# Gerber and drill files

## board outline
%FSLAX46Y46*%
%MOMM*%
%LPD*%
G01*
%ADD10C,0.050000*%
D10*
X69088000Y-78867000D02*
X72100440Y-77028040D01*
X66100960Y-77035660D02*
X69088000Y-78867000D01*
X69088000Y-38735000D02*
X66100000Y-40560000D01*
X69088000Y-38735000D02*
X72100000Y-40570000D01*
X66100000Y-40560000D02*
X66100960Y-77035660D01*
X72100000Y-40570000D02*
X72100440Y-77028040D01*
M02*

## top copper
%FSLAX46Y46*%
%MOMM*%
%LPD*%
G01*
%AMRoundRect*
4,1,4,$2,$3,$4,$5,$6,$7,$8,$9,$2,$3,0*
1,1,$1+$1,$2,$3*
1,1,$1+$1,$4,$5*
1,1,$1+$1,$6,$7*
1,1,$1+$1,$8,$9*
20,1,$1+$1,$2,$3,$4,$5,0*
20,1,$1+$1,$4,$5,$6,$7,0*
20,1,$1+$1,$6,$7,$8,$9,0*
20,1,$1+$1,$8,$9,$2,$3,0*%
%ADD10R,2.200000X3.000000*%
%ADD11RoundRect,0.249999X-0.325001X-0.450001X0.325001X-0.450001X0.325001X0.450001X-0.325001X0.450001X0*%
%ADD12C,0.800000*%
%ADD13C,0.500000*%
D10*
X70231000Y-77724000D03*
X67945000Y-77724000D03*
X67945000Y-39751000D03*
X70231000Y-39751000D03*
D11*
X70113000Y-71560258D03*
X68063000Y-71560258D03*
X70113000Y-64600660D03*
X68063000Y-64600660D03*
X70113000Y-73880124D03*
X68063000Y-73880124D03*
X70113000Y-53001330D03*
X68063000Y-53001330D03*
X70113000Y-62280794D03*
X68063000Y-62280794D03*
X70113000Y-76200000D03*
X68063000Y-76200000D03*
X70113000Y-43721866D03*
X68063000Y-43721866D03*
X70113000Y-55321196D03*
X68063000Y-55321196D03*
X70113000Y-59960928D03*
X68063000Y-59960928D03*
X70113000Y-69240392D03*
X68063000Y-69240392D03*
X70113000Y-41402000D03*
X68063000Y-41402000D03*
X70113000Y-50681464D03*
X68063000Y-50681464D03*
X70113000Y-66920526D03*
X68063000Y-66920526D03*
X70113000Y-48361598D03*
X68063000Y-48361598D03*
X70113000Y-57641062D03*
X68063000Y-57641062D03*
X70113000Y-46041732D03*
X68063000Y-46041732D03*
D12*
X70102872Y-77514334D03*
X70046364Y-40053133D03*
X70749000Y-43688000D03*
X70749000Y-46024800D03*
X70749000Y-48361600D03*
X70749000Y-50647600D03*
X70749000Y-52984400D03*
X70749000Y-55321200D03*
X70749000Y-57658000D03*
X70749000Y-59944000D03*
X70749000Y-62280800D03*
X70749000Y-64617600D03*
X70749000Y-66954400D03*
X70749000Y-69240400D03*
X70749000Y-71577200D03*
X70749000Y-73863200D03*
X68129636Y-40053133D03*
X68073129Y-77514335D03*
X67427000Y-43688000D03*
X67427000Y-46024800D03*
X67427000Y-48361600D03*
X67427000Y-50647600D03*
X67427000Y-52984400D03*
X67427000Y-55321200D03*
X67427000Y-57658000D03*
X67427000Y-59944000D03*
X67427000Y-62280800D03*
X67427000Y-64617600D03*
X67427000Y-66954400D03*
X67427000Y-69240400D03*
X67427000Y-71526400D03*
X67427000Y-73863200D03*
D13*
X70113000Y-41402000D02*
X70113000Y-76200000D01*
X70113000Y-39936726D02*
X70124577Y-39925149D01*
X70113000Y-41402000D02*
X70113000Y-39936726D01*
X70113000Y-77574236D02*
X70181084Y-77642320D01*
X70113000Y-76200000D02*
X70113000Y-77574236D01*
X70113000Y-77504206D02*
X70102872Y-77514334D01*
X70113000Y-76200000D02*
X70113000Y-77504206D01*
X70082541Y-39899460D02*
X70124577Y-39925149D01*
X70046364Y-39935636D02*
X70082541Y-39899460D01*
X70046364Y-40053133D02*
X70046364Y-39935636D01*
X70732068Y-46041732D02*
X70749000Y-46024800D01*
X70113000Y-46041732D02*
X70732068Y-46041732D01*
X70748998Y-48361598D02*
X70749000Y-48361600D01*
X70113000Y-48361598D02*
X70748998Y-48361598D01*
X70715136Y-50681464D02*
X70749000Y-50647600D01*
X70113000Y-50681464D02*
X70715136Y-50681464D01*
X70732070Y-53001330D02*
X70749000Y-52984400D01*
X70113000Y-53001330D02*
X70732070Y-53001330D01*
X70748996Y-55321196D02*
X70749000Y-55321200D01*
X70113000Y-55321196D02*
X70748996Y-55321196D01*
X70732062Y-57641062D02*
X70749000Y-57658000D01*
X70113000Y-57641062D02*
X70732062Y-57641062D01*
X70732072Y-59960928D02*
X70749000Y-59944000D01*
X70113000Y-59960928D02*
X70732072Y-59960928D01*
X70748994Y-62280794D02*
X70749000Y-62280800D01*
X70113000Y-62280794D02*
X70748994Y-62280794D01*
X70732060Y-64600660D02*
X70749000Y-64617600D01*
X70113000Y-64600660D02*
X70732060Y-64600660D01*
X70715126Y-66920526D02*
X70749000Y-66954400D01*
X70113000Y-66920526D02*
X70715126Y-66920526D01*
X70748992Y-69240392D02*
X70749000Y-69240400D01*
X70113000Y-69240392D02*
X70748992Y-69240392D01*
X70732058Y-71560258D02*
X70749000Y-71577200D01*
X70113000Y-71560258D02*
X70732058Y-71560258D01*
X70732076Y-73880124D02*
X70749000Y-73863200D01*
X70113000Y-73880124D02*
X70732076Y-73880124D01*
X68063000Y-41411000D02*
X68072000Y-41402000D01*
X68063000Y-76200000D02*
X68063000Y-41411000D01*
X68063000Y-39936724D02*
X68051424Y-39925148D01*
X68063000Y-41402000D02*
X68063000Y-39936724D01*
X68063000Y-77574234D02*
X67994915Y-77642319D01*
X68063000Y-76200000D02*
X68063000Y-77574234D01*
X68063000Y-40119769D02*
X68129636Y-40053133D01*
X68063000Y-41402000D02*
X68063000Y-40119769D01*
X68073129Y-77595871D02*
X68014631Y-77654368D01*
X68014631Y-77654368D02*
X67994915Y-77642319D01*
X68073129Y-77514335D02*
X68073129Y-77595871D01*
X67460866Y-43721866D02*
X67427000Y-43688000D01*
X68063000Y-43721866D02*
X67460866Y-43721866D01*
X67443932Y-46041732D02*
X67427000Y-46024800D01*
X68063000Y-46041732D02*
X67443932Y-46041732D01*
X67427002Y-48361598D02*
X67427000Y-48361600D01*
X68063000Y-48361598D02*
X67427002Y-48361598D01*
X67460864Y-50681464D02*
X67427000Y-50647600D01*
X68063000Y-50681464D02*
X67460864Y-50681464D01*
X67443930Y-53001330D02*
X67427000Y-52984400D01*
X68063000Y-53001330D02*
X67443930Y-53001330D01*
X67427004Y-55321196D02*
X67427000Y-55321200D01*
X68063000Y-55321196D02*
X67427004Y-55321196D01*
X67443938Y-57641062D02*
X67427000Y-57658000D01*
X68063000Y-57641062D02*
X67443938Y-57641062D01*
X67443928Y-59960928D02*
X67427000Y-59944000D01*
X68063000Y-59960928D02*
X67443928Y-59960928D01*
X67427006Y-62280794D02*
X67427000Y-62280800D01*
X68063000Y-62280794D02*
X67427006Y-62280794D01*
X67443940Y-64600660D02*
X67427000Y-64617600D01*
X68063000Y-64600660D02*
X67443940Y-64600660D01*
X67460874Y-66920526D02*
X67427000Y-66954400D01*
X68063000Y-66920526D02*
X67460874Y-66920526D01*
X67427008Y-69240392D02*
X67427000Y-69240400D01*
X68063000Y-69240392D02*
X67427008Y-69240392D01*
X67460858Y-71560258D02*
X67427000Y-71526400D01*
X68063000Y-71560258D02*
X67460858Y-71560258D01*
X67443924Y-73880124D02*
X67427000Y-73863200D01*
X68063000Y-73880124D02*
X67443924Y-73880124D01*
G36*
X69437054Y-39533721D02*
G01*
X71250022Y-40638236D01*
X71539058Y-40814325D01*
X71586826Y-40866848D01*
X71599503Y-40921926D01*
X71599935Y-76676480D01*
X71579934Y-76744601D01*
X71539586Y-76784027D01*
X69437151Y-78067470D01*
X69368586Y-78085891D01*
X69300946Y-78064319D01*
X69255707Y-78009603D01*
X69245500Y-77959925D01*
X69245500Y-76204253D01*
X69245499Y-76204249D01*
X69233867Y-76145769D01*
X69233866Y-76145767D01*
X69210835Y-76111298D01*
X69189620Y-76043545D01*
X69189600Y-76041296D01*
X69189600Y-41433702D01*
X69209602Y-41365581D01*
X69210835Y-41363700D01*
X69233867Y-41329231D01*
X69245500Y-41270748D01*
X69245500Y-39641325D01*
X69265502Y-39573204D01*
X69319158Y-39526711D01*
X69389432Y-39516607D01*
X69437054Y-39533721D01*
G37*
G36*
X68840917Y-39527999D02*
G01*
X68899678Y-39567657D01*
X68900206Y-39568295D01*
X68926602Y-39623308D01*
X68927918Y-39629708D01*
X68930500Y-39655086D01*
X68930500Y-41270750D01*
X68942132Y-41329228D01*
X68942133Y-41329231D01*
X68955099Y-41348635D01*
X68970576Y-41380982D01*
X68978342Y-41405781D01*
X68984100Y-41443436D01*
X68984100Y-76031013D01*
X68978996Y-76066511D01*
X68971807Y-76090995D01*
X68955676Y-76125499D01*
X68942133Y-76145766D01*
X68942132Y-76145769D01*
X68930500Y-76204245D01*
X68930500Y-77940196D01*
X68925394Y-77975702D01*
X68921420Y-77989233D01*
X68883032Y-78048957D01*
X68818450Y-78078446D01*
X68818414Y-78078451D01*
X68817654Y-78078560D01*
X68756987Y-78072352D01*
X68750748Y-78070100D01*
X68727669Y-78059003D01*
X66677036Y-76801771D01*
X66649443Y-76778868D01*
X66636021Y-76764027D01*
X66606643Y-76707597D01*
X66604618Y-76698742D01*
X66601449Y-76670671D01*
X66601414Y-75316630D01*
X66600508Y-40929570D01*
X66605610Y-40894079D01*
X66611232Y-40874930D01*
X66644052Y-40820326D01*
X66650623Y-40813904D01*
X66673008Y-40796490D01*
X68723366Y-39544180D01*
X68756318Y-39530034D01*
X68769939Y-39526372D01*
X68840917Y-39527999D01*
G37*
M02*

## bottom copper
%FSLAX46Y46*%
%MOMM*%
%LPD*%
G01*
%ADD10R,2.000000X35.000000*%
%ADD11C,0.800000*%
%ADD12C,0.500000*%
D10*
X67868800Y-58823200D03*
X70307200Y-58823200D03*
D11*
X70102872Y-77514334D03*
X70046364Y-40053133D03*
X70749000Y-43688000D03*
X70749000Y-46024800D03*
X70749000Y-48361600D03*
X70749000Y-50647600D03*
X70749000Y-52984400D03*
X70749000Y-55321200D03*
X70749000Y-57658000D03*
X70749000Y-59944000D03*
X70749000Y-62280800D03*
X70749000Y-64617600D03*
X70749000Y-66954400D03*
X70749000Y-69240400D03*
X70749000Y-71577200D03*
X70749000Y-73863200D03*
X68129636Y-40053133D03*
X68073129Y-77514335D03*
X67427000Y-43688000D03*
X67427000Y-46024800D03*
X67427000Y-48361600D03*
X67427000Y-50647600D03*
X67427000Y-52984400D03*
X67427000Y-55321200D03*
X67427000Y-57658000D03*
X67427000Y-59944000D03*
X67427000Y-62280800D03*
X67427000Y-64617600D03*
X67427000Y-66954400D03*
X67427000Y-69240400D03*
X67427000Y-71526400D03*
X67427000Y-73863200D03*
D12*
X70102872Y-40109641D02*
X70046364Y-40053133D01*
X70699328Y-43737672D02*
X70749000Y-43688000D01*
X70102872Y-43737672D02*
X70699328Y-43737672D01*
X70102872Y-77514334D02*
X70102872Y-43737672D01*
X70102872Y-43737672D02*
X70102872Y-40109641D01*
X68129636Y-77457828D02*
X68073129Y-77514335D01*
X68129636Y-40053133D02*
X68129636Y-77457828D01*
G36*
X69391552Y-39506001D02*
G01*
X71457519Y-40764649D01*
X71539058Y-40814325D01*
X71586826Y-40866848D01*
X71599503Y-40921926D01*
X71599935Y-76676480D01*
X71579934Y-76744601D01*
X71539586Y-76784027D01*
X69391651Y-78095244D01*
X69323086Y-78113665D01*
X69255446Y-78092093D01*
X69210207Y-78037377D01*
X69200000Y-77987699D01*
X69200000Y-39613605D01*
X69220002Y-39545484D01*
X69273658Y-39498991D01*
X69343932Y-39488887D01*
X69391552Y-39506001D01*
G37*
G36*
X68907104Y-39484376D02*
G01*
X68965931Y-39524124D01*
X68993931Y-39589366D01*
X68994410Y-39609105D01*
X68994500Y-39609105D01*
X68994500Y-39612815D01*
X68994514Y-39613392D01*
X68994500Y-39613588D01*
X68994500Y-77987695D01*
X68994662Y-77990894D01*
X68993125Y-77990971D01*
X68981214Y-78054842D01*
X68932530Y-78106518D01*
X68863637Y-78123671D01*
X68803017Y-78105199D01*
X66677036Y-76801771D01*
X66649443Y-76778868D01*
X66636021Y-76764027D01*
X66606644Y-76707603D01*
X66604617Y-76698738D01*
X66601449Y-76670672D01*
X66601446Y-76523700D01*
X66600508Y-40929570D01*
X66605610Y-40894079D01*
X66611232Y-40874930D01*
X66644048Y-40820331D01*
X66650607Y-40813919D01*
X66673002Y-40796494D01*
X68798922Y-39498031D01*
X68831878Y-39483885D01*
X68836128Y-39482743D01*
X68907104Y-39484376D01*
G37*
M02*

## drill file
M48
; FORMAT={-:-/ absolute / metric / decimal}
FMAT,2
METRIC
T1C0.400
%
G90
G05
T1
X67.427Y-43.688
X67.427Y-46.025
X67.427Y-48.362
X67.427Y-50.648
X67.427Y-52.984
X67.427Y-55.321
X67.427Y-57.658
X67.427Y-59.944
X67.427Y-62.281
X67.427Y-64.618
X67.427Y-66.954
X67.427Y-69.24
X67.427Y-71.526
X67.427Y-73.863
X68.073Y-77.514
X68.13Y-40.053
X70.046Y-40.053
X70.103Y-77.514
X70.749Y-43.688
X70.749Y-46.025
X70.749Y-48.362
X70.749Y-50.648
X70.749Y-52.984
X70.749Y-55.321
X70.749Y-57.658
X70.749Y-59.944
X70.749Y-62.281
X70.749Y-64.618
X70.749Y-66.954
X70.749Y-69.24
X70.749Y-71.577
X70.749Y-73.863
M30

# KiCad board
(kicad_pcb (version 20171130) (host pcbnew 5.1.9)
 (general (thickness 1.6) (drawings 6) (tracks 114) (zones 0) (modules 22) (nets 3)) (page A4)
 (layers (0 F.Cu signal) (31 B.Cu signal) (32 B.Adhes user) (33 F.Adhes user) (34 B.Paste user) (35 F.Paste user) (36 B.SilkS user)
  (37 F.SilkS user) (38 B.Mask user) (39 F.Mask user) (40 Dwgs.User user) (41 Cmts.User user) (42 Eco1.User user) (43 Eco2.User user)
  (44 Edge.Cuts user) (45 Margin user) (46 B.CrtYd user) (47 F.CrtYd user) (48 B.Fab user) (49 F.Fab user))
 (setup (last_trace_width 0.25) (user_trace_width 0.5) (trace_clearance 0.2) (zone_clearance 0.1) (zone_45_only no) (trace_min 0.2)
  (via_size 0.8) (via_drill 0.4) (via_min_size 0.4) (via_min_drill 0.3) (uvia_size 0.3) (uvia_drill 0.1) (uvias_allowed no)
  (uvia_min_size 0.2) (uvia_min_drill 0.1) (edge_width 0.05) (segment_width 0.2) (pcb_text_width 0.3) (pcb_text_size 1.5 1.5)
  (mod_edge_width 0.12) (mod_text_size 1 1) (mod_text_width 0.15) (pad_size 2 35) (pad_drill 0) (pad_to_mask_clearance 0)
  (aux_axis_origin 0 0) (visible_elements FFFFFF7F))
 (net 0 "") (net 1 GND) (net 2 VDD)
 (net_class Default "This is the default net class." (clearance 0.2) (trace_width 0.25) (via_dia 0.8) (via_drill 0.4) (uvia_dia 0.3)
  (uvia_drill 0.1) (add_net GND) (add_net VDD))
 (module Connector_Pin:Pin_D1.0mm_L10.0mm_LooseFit (layer B.Cu) (at 67.8688 58.8232)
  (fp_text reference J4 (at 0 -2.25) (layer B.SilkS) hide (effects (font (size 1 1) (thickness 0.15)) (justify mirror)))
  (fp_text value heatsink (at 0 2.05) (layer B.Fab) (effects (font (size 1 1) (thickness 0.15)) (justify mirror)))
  (pad 1 connect rect (at 0 0) (size 2 35) (layers B.Cu B.Mask) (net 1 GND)))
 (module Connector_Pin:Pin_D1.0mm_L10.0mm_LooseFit (layer B.Cu) (at 70.3072 58.8232)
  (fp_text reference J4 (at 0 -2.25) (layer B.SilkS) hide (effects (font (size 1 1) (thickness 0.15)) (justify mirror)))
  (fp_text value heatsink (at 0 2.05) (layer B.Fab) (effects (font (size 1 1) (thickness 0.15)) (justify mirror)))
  (pad 1 connect rect (at 0 0) (size 2 35) (layers B.Cu B.Mask) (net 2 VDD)))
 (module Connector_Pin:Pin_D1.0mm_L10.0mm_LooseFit (layer F.Cu) (at 70.231 77.724)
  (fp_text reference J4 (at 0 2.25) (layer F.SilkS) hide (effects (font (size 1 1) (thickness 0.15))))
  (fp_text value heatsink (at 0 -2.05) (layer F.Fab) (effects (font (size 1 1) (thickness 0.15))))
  (pad 1 connect rect (at 0 0) (size 2.2 3) (layers F.Cu F.Mask) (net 2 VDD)))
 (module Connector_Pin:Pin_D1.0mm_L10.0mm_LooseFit (layer F.Cu) (at 67.945 77.724)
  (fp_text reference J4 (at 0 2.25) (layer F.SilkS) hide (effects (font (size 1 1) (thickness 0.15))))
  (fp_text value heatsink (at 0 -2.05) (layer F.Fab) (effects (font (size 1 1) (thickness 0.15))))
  (pad 1 connect rect (at 0 0) (size 2.2 3) (layers F.Cu F.Mask) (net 1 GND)))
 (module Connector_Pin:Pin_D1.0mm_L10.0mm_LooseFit (layer F.Cu) (at 67.945 39.751)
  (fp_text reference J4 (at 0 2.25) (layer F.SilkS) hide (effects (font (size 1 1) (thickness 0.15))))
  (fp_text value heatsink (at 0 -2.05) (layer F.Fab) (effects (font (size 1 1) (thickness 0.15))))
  (pad 1 connect rect (at 0 0) (size 2.2 3) (layers F.Cu F.Mask) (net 1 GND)))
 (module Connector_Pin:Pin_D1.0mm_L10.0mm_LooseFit (layer F.Cu) (at 70.231 39.751)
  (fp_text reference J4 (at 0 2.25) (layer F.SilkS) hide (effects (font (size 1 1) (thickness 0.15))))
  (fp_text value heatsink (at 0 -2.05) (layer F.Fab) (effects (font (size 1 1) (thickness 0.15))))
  (pad 1 connect rect (at 0 0) (size 2.2 3) (layers F.Cu F.Mask) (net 2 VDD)))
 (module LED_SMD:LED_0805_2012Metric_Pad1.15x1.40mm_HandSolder (layer F.Cu) (at 69.088 71.560258)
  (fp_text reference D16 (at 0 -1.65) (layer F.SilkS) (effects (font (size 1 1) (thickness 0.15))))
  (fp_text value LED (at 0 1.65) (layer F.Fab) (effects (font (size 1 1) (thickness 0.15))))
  (pad 2 smd roundrect (at 1.025 0) (size 1.15 1.4) (layers F.Cu F.Paste F.Mask) (roundrect_rratio 0.2173904347826087) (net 2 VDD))
  (pad 1 smd roundrect (at -1.025 0) (size 1.15 1.4) (layers F.Cu F.Paste F.Mask) (roundrect_rratio 0.2173904347826087) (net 1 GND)))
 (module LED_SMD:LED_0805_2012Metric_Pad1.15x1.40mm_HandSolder (layer F.Cu) (at 69.088 64.60066)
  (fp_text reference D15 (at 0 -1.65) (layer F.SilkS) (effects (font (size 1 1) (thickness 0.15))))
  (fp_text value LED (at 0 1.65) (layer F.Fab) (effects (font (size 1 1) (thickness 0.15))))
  (pad 2 smd roundrect (at 1.025 0) (size 1.15 1.4) (layers F.Cu F.Paste F.Mask) (roundrect_rratio 0.2173904347826087) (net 2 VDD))
  (pad 1 smd roundrect (at -1.025 0) (size 1.15 1.4) (layers F.Cu F.Paste F.Mask) (roundrect_rratio 0.2173904347826087) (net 1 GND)))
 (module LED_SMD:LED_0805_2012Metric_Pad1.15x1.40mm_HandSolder (layer F.Cu) (at 69.088 73.880124)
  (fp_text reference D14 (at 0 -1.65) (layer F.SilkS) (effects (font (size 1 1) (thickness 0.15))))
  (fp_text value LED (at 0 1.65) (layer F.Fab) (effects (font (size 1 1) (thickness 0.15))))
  (pad 2 smd roundrect (at 1.025 0) (size 1.15 1.4) (layers F.Cu F.Paste F.Mask) (roundrect_rratio 0.2173904347826087) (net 2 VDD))
  (pad 1 smd roundrect (at -1.025 0) (size 1.15 1.4) (layers F.Cu F.Paste F.Mask) (roundrect_rratio 0.2173904347826087) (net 1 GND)))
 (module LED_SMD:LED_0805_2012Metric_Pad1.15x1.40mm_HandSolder (layer F.Cu) (at 69.088 53.00133)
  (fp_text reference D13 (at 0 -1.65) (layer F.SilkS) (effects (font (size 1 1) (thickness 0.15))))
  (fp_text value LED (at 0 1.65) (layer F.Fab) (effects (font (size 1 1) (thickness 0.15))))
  (pad 2 smd roundrect (at 1.025 0) (size 1.15 1.4) (layers F.Cu F.Paste F.Mask) (roundrect_rratio 0.2173904347826087) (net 2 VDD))
  (pad 1 smd roundrect (at -1.025 0) (size 1.15 1.4) (layers F.Cu F.Paste F.Mask) (roundrect_rratio 0.2173904347826087) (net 1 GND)))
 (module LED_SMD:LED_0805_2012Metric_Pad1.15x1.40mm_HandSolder (layer F.Cu) (at 69.088 62.280794)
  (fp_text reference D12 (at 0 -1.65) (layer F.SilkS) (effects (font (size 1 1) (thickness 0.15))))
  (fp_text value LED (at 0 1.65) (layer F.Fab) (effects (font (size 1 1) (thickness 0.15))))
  (pad 2 smd roundrect (at 1.025 0) (size 1.15 1.4) (layers F.Cu F.Paste F.Mask) (roundrect_rratio 0.2173904347826087) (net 2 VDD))
  (pad 1 smd roundrect (at -1.025 0) (size 1.15 1.4) (layers F.Cu F.Paste F.Mask) (roundrect_rratio 0.2173904347826087) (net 1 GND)))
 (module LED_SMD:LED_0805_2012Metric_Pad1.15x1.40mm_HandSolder (layer F.Cu) (at 69.088 76.2)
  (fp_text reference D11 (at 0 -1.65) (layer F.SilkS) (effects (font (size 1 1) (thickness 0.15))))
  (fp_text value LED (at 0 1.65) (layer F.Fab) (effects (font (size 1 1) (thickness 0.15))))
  (pad 2 smd roundrect (at 1.025 0) (size 1.15 1.4) (layers F.Cu F.Paste F.Mask) (roundrect_rratio 0.2173904347826087) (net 2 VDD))
  (pad 1 smd roundrect (at -1.025 0) (size 1.15 1.4) (layers F.Cu F.Paste F.Mask) (roundrect_rratio 0.2173904347826087) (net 1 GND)))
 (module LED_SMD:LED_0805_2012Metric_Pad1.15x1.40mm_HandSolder (layer F.Cu) (at 69.088 43.721866)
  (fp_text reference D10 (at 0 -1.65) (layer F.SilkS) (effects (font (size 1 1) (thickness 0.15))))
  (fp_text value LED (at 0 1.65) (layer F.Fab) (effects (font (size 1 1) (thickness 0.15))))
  (pad 2 smd roundrect (at 1.025 0) (size 1.15 1.4) (layers F.Cu F.Paste F.Mask) (roundrect_rratio 0.2173904347826087) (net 2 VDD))
  (pad 1 smd roundrect (at -1.025 0) (size 1.15 1.4) (layers F.Cu F.Paste F.Mask) (roundrect_rratio 0.2173904347826087) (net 1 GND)))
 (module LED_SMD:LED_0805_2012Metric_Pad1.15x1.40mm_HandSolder (layer F.Cu) (at 69.088 55.321196)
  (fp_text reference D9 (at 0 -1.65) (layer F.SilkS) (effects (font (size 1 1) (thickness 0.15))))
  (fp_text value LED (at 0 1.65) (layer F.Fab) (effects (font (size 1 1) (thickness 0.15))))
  (pad 2 smd roundrect (at 1.025 0) (size 1.15 1.4) (layers F.Cu F.Paste F.Mask) (roundrect_rratio 0.2173904347826087) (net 2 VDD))
  (pad 1 smd roundrect (at -1.025 0) (size 1.15 1.4) (layers F.Cu F.Paste F.Mask) (roundrect_rratio 0.2173904347826087) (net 1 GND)))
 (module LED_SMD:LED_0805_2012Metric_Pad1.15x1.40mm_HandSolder (layer F.Cu) (at 69.088 59.960928)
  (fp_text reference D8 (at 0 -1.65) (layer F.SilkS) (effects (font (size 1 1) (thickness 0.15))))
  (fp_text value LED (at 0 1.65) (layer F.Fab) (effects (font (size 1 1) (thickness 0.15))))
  (pad 2 smd roundrect (at 1.025 0) (size 1.15 1.4) (layers F.Cu F.Paste F.Mask) (roundrect_rratio 0.2173904347826087) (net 2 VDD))
  (pad 1 smd roundrect (at -1.025 0) (size 1.15 1.4) (layers F.Cu F.Paste F.Mask) (roundrect_rratio 0.2173904347826087) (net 1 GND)))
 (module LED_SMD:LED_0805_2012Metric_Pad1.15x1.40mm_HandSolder (layer F.Cu) (at 69.088 69.240392)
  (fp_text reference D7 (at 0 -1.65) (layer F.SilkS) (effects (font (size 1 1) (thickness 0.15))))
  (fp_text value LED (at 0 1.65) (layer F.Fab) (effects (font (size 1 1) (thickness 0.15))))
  (pad 2 smd roundrect (at 1.025 0) (size 1.15 1.4) (layers F.Cu F.Paste F.Mask) (roundrect_rratio 0.2173904347826087) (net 2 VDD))
  (pad 1 smd roundrect (at -1.025 0) (size 1.15 1.4) (layers F.Cu F.Paste F.Mask) (roundrect_rratio 0.2173904347826087) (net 1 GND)))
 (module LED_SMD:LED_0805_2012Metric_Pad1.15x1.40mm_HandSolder (layer F.Cu) (at 69.088 41.402)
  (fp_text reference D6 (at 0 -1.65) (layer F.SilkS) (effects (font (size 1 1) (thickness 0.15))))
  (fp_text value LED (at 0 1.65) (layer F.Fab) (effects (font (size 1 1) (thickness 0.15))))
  (pad 2 smd roundrect (at 1.025 0) (size 1.15 1.4) (layers F.Cu F.Paste F.Mask) (roundrect_rratio 0.2173904347826087) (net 2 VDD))
  (pad 1 smd roundrect (at -1.025 0) (size 1.15 1.4) (layers F.Cu F.Paste F.Mask) (roundrect_rratio 0.2173904347826087) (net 1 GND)))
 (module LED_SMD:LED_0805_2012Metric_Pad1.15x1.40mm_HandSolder (layer F.Cu) (at 69.088 50.681464)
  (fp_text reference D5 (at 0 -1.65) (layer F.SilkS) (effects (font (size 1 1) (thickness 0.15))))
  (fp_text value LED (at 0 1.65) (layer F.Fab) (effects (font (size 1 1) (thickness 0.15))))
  (pad 2 smd roundrect (at 1.025 0) (size 1.15 1.4) (layers F.Cu F.Paste F.Mask) (roundrect_rratio 0.2173904347826087) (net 2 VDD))
  (pad 1 smd roundrect (at -1.025 0) (size 1.15 1.4) (layers F.Cu F.Paste F.Mask) (roundrect_rratio 0.2173904347826087) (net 1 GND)))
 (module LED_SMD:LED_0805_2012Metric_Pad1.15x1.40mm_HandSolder (layer F.Cu) (at 69.088 66.920526)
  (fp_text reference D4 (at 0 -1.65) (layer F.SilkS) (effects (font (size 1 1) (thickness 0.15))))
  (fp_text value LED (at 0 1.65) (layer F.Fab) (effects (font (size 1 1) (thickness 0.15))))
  (pad 2 smd roundrect (at 1.025 0) (size 1.15 1.4) (layers F.Cu F.Paste F.Mask) (roundrect_rratio 0.2173904347826087) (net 2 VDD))
  (pad 1 smd roundrect (at -1.025 0) (size 1.15 1.4) (layers F.Cu F.Paste F.Mask) (roundrect_rratio 0.2173904347826087) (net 1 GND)))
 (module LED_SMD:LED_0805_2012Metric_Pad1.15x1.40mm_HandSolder (layer F.Cu) (at 69.088 48.361598)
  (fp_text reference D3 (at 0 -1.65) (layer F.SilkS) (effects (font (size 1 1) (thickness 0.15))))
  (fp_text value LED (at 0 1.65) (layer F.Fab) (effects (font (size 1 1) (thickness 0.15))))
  (pad 2 smd roundrect (at 1.025 0) (size 1.15 1.4) (layers F.Cu F.Paste F.Mask) (roundrect_rratio 0.2173904347826087) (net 2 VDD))
  (pad 1 smd roundrect (at -1.025 0) (size 1.15 1.4) (layers F.Cu F.Paste F.Mask) (roundrect_rratio 0.2173904347826087) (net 1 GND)))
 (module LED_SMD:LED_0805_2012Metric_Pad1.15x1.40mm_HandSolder (layer F.Cu) (at 69.088 57.641062)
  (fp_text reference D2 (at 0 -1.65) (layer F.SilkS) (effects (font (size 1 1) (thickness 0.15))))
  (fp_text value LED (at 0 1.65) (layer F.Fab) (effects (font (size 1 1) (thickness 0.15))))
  (pad 2 smd roundrect (at 1.025 0) (size 1.15 1.4) (layers F.Cu F.Paste F.Mask) (roundrect_rratio 0.2173904347826087) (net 2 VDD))
  (pad 1 smd roundrect (at -1.025 0) (size 1.15 1.4) (layers F.Cu F.Paste F.Mask) (roundrect_rratio 0.2173904347826087) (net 1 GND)))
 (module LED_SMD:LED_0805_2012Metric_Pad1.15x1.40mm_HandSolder (layer F.Cu) (at 69.088 46.041732)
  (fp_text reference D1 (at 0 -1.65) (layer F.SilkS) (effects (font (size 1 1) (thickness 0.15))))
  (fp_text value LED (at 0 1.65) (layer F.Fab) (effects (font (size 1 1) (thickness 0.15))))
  (pad 2 smd roundrect (at 1.025 0) (size 1.15 1.4) (layers F.Cu F.Paste F.Mask) (roundrect_rratio 0.2173904347826087) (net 2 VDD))
  (pad 1 smd roundrect (at -1.025 0) (size 1.15 1.4) (layers F.Cu F.Paste F.Mask) (roundrect_rratio 0.2173904347826087) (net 1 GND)))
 (gr_line (start 69.088 78.867) (end 72.10044 77.02804) (layer Edge.Cuts) (width 0.05))
 (gr_line (start 66.10096 77.03566) (end 69.088 78.867) (layer Edge.Cuts) (width 0.05))
 (gr_line (start 69.088 38.735) (end 66.1 40.56) (layer Edge.Cuts) (width 0.05))
 (gr_line (start 69.088 38.735) (end 72.1 40.57) (layer Edge.Cuts) (width 0.05))
 (gr_line (start 66.1 40.56) (end 66.10096 77.03566) (layer Edge.Cuts) (width 0.05))
 (gr_line (start 72.1 40.57) (end 72.10044 77.02804) (layer Edge.Cuts) (width 0.05))
 (segment (start 70.113 41.402) (end 70.113 76.2) (width 0.5) (layer F.Cu) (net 2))
 (segment (start 70.113 39.936726) (end 70.124577 39.925149) (width 0.5) (layer F.Cu) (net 2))
 (segment (start 70.113 41.402) (end 70.113 39.936726) (width 0.5) (layer F.Cu) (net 2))
 (segment (start 70.113 77.574236) (end 70.181084 77.64232) (width 0.5) (layer F.Cu) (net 2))
 (segment (start 70.113 76.2) (end 70.113 77.574236) (width 0.5) (layer F.Cu) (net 2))
 (via (at 70.102872 77.514334) (size 0.8) (drill 0.4) (layers F.Cu B.Cu) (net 2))
 (segment (start 70.113 77.504206) (end 70.102872 77.514334) (width 0.5) (layer F.Cu) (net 2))
 (segment (start 70.113 76.2) (end 70.113 77.504206) (width 0.5) (layer F.Cu) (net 2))
 (via (at 70.046364 40.053133) (size 0.8) (drill 0.4) (layers F.Cu B.Cu) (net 2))
 (segment (start 70.102872 40.109641) (end 70.046364 40.053133) (width 0.5) (layer B.Cu) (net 2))
 (segment (start 70.082541 39.89946) (end 70.124577 39.925149) (width 0.5) (layer F.Cu) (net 2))
 (segment (start 70.046364 39.935636) (end 70.082541 39.89946) (width 0.5) (layer F.Cu) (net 2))
 (segment (start 70.046364 40.053133) (end 70.046364 39.935636) (width 0.5) (layer F.Cu) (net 2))
 (via (at 70.749 43.688) (size 0.8) (drill 0.4) (layers F.Cu B.Cu) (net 2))
 (segment (start 70.699328 43.737672) (end 70.749 43.688) (width 0.5) (layer B.Cu) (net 2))
 (segment (start 70.102872 43.737672) (end 70.699328 43.737672) (width 0.5) (layer B.Cu) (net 2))
 (segment (start 70.102872 77.514334) (end 70.102872 43.737672) (width 0.5) (layer B.Cu) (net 2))
 (segment (start 70.102872 43.737672) (end 70.102872 40.109641) (width 0.5) (layer B.Cu) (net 2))
 (via (at 70.749 46.0248) (size 0.8) (drill 0.4) (layers F.Cu B.Cu) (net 2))
 (segment (start 70.732068 46.041732) (end 70.749 46.0248) (width 0.5) (layer F.Cu) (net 2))
 (segment (start 70.113 46.041732) (end 70.732068 46.041732) (width 0.5) (layer F.Cu) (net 2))
 (segment (start 70.748998 48.361598) (end 70.749 48.3616) (width 0.5) (layer F.Cu) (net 2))
 (via (at 70.749 48.3616) (size 0.8) (drill 0.4) (layers F.Cu B.Cu) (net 2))
 (segment (start 70.113 48.361598) (end 70.748998 48.361598) (width 0.5) (layer F.Cu) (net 2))
 (via (at 70.749 50.6476) (size 0.8) (drill 0.4) (layers F.Cu B.Cu) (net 2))
 (segment (start 70.715136 50.681464) (end 70.749 50.6476) (width 0.5) (layer F.Cu) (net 2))
 (segment (start 70.113 50.681464) (end 70.715136 50.681464) (width 0.5) (layer F.Cu) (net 2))
 (via (at 70.749 52.9844) (size 0.8) (drill 0.4) (layers F.Cu B.Cu) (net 2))
 (segment (start 70.73207 53.00133) (end 70.749 52.9844) (width 0.5) (layer F.Cu) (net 2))
 (segment (start 70.113 53.00133) (end 70.73207 53.00133) (width 0.5) (layer F.Cu) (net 2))
 (via (at 70.749 55.3212) (size 0.8) (drill 0.4) (layers F.Cu B.Cu) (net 2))
 (segment (start 70.748996 55.321196) (end 70.749 55.3212) (width 0.5) (layer F.Cu) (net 2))
 (segment (start 70.113 55.321196) (end 70.748996 55.321196) (width 0.5) (layer F.Cu) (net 2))
 (via (at 70.749 57.658) (size 0.8) (drill 0.4) (layers F.Cu B.Cu) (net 2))
 (segment (start 70.732062 57.641062) (end 70.749 57.658) (width 0.5) (layer F.Cu) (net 2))
 (segment (start 70.113 57.641062) (end 70.732062 57.641062) (width 0.5) (layer F.Cu) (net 2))
 (via (at 70.749 59.944) (size 0.8) (drill 0.4) (layers F.Cu B.Cu) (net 2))
 (segment (start 70.732072 59.960928) (end 70.749 59.944) (width 0.5) (layer F.Cu) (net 2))
 (segment (start 70.113 59.960928) (end 70.732072 59.960928) (width 0.5) (layer F.Cu) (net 2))
 (via (at 70.749 62.2808) (size 0.8) (drill 0.4) (layers F.Cu B.Cu) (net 2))
 (segment (start 70.748994 62.280794) (end 70.749 62.2808) (width 0.5) (layer F.Cu) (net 2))
 (segment (start 70.113 62.280794) (end 70.748994 62.280794) (width 0.5) (layer F.Cu) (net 2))
 (via (at 70.749 64.6176) (size 0.8) (drill 0.4) (layers F.Cu B.Cu) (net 2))
 (segment (start 70.73206 64.60066) (end 70.749 64.6176) (width 0.5) (layer F.Cu) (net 2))
 (segment (start 70.113 64.60066) (end 70.73206 64.60066) (width 0.5) (layer F.Cu) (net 2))
 (via (at 70.749 66.9544) (size 0.8) (drill 0.4) (layers F.Cu B.Cu) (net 2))
 (segment (start 70.715126 66.920526) (end 70.749 66.9544) (width 0.5) (layer F.Cu) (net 2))
 (segment (start 70.113 66.920526) (end 70.715126 66.920526) (width 0.5) (layer F.Cu) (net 2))
 (via (at 70.749 69.2404) (size 0.8) (drill 0.4) (layers F.Cu B.Cu) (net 2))
 (segment (start 70.748992 69.240392) (end 70.749 69.2404) (width 0.5) (layer F.Cu) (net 2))
 (segment (start 70.113 69.240392) (end 70.748992 69.240392) (width 0.5) (layer F.Cu) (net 2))
 (via (at 70.749 71.5772) (size 0.8) (drill 0.4) (layers F.Cu B.Cu) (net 2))
 (segment (start 70.732058 71.560258) (end 70.749 71.5772) (width 0.5) (layer F.Cu) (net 2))
 (segment (start 70.113 71.560258) (end 70.732058 71.560258) (width 0.5) (layer F.Cu) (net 2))
 (via (at 70.749 73.8632) (size 0.8) (drill 0.4) (layers F.Cu B.Cu) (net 2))
 (segment (start 70.732076 73.880124) (end 70.749 73.8632) (width 0.5) (layer F.Cu) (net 2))
 (segment (start 70.113 73.880124) (end 70.732076 73.880124) (width 0.5) (layer F.Cu) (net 2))
 (segment (start 68.063 41.411) (end 68.072 41.402) (width 0.5) (layer F.Cu) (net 1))
 (segment (start 68.063 76.2) (end 68.063 41.411) (width 0.5) (layer F.Cu) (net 1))
 (segment (start 68.063 39.936724) (end 68.051424 39.925148) (width 0.5) (layer F.Cu) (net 1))
 (segment (start 68.063 41.402) (end 68.063 39.936724) (width 0.5) (layer F.Cu) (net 1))
 (segment (start 68.063 77.574234) (end 67.994915 77.642319) (width 0.5) (layer F.Cu) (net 1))
 (segment (start 68.063 76.2) (end 68.063 77.574234) (width 0.5) (layer F.Cu) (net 1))
 (via (at 68.129636 40.053133) (size 0.8) (drill 0.4) (layers F.Cu B.Cu) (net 1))
 (segment (start 68.063 40.119769) (end 68.129636 40.053133) (width 0.5) (layer F.Cu) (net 1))
 (segment (start 68.063 41.402) (end 68.063 40.119769) (width 0.5) (layer F.Cu) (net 1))
 (via (at 68.073129 77.514335) (size 0.8) (drill 0.4) (layers F.Cu B.Cu) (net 1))
 (segment (start 68.129636 77.457828) (end 68.073129 77.514335) (width 0.5) (layer B.Cu) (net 1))
 (segment (start 68.129636 40.053133) (end 68.129636 77.457828) (width 0.5) (layer B.Cu) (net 1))
 (segment (start 68.073129 77.595871) (end 68.014631 77.654368) (width 0.5) (layer F.Cu) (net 1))
 (segment (start 68.014631 77.654368) (end 67.994915 77.642319) (width 0.5) (layer F.Cu) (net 1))
 (segment (start 68.073129 77.514335) (end 68.073129 77.595871) (width 0.5) (layer F.Cu) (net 1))
 (segment (start 67.460866 43.721866) (end 67.427 43.688) (width 0.5) (layer F.Cu) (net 1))
 (via (at 67.427 43.688) (size 0.8) (drill 0.4) (layers F.Cu B.Cu) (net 1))
 (segment (start 68.063 43.721866) (end 67.460866 43.721866) (width 0.5) (layer F.Cu) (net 1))
 (via (at 67.427 46.0248) (size 0.8) (drill 0.4) (layers F.Cu B.Cu) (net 1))
 (segment (start 67.443932 46.041732) (end 67.427 46.0248) (width 0.5) (layer F.Cu) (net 1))
 (segment (start 68.063 46.041732) (end 67.443932 46.041732) (width 0.5) (layer F.Cu) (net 1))
 (via (at 67.427 48.3616) (size 0.8) (drill 0.4) (layers F.Cu B.Cu) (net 1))
 (segment (start 67.427002 48.361598) (end 67.427 48.3616) (width 0.5) (layer F.Cu) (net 1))
 (segment (start 68.063 48.361598) (end 67.427002 48.361598) (width 0.5) (layer F.Cu) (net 1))
 (via (at 67.427 50.6476) (size 0.8) (drill 0.4) (layers F.Cu B.Cu) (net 1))
 (segment (start 67.460864 50.681464) (end 67.427 50.6476) (width 0.5) (layer F.Cu) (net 1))
 (segment (start 68.063 50.681464) (end 67.460864 50.681464) (width 0.5) (layer F.Cu) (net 1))
 (via (at 67.427 52.9844) (size 0.8) (drill 0.4) (layers F.Cu B.Cu) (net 1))
 (segment (start 67.44393 53.00133) (end 67.427 52.9844) (width 0.5) (layer F.Cu) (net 1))
 (segment (start 68.063 53.00133) (end 67.44393 53.00133) (width 0.5) (layer F.Cu) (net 1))
 (via (at 67.427 55.3212) (size 0.8) (drill 0.4) (layers F.Cu B.Cu) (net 1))
 (segment (start 67.427004 55.321196) (end 67.427 55.3212) (width 0.5) (layer F.Cu) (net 1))
 (segment (start 68.063 55.321196) (end 67.427004 55.321196) (width 0.5) (layer F.Cu) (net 1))
 (via (at 67.427 57.658) (size 0.8) (drill 0.4) (layers F.Cu B.Cu) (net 1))
 (segment (start 67.443938 57.641062) (end 67.427 57.658) (width 0.5) (layer F.Cu) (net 1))
 (segment (start 68.063 57.641062) (end 67.443938 57.641062) (width 0.5) (layer F.Cu) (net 1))
 (via (at 67.427 59.944) (size 0.8) (drill 0.4) (layers F.Cu B.Cu) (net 1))
 (segment (start 67.443928 59.960928) (end 67.427 59.944) (width 0.5) (layer F.Cu) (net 1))
 (segment (start 68.063 59.960928) (end 67.443928 59.960928) (width 0.5) (layer F.Cu) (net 1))
 (via (at 67.427 62.2808) (size 0.8) (drill 0.4) (layers F.Cu B.Cu) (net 1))
 (segment (start 67.427006 62.280794) (end 67.427 62.2808) (width 0.5) (layer F.Cu) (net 1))
 (segment (start 68.063 62.280794) (end 67.427006 62.280794) (width 0.5) (layer F.Cu) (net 1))
 (via (at 67.427 64.6176) (size 0.8) (drill 0.4) (layers F.Cu B.Cu) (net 1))
 (segment (start 67.44394 64.60066) (end 67.427 64.6176) (width 0.5) (layer F.Cu) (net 1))
 (segment (start 68.063 64.60066) (end 67.44394 64.60066) (width 0.5) (layer F.Cu) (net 1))
 (via (at 67.427 66.9544) (size 0.8) (drill 0.4) (layers F.Cu B.Cu) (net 1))
 (segment (start 67.460874 66.920526) (end 67.427 66.9544) (width 0.5) (layer F.Cu) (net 1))
 (segment (start 68.063 66.920526) (end 67.460874 66.920526) (width 0.5) (layer F.Cu) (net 1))
 (via (at 67.427 69.2404) (size 0.8) (drill 0.4) (layers F.Cu B.Cu) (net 1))
 (segment (start 67.427008 69.240392) (end 67.427 69.2404) (width 0.5) (layer F.Cu) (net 1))
 (segment (start 68.063 69.240392) (end 67.427008 69.240392) (width 0.5) (layer F.Cu) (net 1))
 (via (at 67.427 71.5264) (size 0.8) (drill 0.4) (layers F.Cu B.Cu) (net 1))
 (segment (start 67.460858 71.560258) (end 67.427 71.5264) (width 0.5) (layer F.Cu) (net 1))
 (segment (start 68.063 71.560258) (end 67.460858 71.560258) (width 0.5) (layer F.Cu) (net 1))
 (via (at 67.427 73.8632) (size 0.8) (drill 0.4) (layers F.Cu B.Cu) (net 1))
 (segment (start 67.443924 73.880124) (end 67.427 73.8632) (width 0.5) (layer F.Cu) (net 1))
 (segment (start 68.063 73.880124) (end 67.443924 73.880124) (width 0.5) (layer F.Cu) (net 1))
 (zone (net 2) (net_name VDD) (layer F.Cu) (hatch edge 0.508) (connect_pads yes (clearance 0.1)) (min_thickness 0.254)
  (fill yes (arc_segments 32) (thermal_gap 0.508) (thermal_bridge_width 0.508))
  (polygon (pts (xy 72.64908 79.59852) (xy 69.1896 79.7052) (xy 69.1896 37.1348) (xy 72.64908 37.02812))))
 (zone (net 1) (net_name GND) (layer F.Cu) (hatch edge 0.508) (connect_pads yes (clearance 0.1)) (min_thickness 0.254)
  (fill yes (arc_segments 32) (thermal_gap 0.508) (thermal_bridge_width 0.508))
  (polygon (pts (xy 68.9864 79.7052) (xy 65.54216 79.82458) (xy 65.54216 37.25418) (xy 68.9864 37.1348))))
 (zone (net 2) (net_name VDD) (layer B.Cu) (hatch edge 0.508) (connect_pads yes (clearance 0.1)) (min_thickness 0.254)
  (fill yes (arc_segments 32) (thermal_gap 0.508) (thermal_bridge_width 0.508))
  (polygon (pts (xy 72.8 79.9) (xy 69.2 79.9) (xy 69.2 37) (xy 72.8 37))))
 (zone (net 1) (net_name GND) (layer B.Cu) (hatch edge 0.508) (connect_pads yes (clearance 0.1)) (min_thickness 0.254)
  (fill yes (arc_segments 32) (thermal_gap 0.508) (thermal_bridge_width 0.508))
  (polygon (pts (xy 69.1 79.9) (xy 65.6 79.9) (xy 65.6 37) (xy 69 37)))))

